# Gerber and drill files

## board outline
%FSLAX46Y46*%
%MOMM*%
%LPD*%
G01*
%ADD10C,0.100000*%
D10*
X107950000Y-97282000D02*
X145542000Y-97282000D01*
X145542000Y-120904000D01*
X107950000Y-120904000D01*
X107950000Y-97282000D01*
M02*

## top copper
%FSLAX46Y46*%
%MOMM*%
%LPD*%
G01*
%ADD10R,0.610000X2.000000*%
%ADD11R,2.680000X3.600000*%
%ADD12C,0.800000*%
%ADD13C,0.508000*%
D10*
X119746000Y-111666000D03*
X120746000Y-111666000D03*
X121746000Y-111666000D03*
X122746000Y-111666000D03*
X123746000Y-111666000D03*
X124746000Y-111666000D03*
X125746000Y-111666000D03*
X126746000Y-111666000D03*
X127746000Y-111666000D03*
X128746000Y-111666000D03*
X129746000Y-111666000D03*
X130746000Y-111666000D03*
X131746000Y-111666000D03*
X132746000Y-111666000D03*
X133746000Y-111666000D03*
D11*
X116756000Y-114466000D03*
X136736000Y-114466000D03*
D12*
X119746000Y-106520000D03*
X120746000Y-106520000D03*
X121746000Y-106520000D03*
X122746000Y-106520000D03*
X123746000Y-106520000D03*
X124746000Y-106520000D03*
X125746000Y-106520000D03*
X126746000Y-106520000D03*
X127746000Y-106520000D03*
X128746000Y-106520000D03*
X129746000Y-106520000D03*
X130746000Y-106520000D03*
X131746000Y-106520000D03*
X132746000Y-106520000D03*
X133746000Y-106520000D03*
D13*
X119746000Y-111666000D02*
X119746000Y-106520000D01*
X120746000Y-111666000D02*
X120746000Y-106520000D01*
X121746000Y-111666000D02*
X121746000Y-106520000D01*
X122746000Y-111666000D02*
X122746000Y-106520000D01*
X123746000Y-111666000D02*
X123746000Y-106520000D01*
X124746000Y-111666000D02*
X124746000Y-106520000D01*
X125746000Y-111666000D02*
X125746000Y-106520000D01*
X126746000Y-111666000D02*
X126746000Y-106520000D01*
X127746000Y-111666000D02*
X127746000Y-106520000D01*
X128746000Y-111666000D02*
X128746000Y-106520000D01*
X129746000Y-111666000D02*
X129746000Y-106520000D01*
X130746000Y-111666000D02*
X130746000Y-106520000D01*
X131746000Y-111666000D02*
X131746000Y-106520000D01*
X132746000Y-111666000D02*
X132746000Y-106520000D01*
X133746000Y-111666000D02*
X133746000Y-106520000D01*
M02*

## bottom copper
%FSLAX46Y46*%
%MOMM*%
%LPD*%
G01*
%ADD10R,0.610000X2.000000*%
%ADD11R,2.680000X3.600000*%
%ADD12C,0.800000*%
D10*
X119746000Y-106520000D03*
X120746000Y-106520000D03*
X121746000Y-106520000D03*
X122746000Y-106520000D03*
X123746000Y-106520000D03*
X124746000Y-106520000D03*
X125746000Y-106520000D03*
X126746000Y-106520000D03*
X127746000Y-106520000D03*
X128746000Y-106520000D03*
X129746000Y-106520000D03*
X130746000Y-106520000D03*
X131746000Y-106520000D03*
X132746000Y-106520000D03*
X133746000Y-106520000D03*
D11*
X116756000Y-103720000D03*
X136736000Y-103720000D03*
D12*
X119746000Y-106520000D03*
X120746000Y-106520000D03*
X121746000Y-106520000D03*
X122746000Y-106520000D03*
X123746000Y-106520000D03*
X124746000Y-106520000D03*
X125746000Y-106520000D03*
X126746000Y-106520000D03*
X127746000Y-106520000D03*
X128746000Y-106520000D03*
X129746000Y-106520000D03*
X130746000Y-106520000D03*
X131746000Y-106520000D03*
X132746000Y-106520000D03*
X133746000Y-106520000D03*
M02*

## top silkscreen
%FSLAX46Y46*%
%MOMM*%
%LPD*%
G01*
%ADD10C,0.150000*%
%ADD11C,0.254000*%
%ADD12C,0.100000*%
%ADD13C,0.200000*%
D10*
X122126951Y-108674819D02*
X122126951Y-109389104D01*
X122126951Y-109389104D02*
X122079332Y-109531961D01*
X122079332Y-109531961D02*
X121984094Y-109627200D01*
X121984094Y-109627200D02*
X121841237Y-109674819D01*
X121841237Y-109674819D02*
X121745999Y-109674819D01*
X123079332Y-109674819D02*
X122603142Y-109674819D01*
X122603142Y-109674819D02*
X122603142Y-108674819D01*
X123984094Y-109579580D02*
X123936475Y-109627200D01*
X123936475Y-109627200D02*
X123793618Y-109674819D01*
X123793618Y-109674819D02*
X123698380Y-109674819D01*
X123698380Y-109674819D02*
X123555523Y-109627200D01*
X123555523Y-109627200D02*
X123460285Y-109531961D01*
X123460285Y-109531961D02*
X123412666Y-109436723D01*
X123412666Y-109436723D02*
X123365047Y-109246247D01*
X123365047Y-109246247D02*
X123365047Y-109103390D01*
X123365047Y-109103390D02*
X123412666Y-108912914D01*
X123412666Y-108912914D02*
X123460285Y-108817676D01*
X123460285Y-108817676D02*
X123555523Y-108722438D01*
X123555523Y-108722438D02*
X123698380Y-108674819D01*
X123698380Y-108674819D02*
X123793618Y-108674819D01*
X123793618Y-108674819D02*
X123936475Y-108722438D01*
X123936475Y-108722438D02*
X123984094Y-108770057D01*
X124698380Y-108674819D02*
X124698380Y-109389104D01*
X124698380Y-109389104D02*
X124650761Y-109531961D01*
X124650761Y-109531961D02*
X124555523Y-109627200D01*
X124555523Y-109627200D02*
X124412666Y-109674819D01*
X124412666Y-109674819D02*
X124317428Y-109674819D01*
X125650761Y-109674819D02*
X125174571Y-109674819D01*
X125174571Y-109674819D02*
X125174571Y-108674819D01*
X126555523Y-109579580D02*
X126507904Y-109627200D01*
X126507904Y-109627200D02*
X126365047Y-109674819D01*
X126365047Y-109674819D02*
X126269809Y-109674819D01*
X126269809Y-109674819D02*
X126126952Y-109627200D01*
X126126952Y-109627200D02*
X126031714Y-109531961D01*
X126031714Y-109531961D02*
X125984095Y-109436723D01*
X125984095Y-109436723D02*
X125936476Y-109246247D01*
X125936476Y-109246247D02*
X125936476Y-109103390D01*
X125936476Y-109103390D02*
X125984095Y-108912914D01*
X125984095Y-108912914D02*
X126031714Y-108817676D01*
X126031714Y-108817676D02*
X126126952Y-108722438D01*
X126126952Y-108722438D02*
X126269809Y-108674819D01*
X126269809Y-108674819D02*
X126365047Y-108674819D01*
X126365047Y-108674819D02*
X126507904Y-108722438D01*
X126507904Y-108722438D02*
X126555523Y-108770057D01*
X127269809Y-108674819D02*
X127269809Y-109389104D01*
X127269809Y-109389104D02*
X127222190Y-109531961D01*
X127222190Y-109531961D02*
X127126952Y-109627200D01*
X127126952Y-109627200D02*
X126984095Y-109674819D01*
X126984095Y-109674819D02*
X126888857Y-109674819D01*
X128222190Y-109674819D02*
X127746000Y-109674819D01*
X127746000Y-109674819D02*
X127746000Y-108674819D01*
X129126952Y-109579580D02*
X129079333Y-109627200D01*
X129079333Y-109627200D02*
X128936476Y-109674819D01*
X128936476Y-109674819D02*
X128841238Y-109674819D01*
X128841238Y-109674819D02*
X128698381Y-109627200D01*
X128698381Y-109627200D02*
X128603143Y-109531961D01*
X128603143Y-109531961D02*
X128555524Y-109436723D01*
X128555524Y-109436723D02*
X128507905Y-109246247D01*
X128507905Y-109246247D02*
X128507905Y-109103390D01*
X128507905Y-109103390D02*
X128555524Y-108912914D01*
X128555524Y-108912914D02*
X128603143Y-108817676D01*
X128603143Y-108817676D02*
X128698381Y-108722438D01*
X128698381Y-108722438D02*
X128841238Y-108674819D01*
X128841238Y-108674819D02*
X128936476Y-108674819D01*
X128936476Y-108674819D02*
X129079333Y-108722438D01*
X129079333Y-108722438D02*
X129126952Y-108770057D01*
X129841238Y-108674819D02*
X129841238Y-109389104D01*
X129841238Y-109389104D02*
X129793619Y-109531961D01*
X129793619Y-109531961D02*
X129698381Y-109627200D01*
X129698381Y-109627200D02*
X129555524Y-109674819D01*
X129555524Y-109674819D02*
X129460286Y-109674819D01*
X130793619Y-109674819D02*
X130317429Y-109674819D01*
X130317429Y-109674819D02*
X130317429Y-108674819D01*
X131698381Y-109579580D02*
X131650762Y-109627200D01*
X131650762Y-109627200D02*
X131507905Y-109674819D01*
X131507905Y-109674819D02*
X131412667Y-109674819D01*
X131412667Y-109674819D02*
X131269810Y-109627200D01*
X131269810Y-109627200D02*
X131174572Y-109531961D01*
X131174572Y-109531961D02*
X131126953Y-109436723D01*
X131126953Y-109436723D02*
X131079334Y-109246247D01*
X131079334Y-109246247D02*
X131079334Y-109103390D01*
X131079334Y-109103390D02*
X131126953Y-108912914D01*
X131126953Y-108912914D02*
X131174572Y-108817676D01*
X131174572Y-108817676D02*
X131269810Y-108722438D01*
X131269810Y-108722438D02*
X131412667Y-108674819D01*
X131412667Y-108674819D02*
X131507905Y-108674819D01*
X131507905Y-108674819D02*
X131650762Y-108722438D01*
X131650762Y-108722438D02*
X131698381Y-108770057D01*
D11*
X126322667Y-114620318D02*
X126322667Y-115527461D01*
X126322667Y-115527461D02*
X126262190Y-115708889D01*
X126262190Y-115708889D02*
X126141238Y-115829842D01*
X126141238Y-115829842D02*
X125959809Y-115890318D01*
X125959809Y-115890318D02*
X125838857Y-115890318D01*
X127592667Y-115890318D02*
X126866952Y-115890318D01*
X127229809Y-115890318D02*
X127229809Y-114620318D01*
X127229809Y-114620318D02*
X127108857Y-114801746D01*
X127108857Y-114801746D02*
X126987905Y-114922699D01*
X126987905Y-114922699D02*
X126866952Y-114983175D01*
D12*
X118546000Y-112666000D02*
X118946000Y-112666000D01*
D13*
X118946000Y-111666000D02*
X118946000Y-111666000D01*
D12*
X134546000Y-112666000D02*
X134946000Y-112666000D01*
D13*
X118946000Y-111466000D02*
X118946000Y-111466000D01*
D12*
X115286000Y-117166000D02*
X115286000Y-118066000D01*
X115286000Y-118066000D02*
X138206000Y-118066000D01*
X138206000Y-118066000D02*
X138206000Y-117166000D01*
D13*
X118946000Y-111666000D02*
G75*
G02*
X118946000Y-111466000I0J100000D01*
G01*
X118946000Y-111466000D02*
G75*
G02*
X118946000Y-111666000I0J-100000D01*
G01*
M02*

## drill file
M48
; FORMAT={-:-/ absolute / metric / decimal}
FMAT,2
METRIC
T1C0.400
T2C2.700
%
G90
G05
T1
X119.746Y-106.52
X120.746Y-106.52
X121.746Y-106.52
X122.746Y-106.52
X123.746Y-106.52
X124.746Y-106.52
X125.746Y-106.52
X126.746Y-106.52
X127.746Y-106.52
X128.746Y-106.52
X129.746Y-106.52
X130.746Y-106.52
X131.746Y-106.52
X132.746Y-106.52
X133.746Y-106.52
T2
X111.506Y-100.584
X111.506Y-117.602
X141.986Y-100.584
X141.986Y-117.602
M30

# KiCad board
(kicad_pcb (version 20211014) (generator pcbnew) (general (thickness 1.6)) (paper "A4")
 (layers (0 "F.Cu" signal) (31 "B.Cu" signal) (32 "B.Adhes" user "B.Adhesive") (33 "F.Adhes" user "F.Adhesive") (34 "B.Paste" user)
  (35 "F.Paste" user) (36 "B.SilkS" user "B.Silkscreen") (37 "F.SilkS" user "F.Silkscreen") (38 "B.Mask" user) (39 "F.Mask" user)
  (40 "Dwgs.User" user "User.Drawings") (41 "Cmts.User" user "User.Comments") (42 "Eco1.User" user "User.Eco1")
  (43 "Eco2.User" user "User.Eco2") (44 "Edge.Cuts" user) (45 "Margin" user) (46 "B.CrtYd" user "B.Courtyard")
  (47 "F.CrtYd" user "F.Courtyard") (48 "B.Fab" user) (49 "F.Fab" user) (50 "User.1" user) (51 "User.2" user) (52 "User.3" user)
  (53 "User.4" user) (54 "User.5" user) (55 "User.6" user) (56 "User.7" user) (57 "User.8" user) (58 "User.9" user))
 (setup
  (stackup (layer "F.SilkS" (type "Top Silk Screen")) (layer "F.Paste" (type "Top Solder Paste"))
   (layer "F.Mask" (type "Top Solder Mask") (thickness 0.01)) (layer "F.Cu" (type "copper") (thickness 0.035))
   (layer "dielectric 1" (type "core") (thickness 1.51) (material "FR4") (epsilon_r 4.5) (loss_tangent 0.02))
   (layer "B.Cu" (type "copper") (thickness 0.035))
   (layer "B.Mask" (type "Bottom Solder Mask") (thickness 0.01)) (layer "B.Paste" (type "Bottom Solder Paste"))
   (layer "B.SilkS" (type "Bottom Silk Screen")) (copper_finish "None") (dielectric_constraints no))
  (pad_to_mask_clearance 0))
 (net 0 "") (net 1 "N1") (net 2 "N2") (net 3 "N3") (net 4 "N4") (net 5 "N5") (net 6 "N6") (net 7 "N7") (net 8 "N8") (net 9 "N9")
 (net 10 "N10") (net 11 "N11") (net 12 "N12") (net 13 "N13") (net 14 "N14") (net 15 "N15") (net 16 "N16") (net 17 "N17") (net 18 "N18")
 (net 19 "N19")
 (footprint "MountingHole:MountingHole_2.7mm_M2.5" (layer "F.Cu") (at 141.986 100.584)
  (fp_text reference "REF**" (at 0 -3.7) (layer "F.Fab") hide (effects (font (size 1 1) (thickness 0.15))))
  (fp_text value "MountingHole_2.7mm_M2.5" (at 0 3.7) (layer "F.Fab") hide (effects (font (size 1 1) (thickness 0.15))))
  (pad "" np_thru_hole circle locked (at 0 0) (size 2.7 2.7) (drill 2.7) (layers *.Cu *.Mask)))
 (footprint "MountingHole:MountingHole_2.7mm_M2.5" (layer "F.Cu") (at 141.986 117.602)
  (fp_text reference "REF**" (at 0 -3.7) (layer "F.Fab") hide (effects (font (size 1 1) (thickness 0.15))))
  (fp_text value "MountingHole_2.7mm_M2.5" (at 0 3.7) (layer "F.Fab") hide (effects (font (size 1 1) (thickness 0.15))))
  (pad "" np_thru_hole circle locked (at 0 0) (size 2.7 2.7) (drill 2.7) (layers *.Cu *.Mask)))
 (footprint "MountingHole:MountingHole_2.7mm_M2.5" (layer "F.Cu") (at 111.506 100.584)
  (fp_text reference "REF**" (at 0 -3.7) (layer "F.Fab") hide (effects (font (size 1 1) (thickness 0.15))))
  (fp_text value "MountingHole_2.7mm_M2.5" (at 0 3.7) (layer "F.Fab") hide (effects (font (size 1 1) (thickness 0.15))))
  (pad "" np_thru_hole circle locked (at 0 0) (size 2.7 2.7) (drill 2.7) (layers *.Cu *.Mask)))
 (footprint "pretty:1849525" (layer "F.Cu") (at 126.746 115.316)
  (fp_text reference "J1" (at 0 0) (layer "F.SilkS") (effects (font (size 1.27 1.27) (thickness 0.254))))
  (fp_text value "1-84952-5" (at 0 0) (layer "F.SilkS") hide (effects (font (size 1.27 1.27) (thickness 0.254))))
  (fp_line (start -8.2 -2.65) (end -7.8 -2.65) (layer "F.SilkS") (width 0.1))
  (fp_line (start -7.8 -3.65) (end -7.8 -3.65) (layer "F.SilkS") (width 0.2))
  (fp_line (start 7.8 -2.65) (end 8.2 -2.65) (layer "F.SilkS") (width 0.1))
  (fp_line (start -7.8 -3.85) (end -7.8 -3.85) (layer "F.SilkS") (width 0.2))
  (fp_line (start -11.46 1.85) (end -11.46 2.75) (layer "F.SilkS") (width 0.1))
  (fp_line (start -11.46 2.75) (end 11.46 2.75) (layer "F.SilkS") (width 0.1))
  (fp_line (start 11.46 2.75) (end 11.46 1.85) (layer "F.SilkS") (width 0.1))
  (fp_arc (start -7.8 -3.65) (mid -7.9 -3.75) (end -7.8 -3.85) (layer "F.SilkS") (width 0.2))
  (fp_arc (start -7.8 -3.85) (mid -7.7 -3.75) (end -7.8 -3.65) (layer "F.SilkS") (width 0.2))
  (pad "1" smd rect locked (at -7 -3.65) (size 0.61 2) (layers "F.Cu" "F.Paste" "F.Mask") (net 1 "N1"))
  (pad "2" smd rect locked (at -6 -3.65) (size 0.61 2) (layers "F.Cu" "F.Paste" "F.Mask") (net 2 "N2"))
  (pad "3" smd rect locked (at -5 -3.65) (size 0.61 2) (layers "F.Cu" "F.Paste" "F.Mask") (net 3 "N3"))
  (pad "4" smd rect locked (at -4 -3.65) (size 0.61 2) (layers "F.Cu" "F.Paste" "F.Mask") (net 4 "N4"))
  (pad "5" smd rect locked (at -3 -3.65) (size 0.61 2) (layers "F.Cu" "F.Paste" "F.Mask") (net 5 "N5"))
  (pad "6" smd rect locked (at -2 -3.65) (size 0.61 2) (layers "F.Cu" "F.Paste" "F.Mask") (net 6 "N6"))
  (pad "7" smd rect locked (at -1 -3.65) (size 0.61 2) (layers "F.Cu" "F.Paste" "F.Mask") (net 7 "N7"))
  (pad "8" smd rect locked (at 0 -3.65) (size 0.61 2) (layers "F.Cu" "F.Paste" "F.Mask") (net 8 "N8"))
  (pad "9" smd rect locked (at 1 -3.65) (size 0.61 2) (layers "F.Cu" "F.Paste" "F.Mask") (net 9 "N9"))
  (pad "10" smd rect locked (at 2 -3.65) (size 0.61 2) (layers "F.Cu" "F.Paste" "F.Mask") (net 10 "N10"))
  (pad "11" smd rect locked (at 3 -3.65) (size 0.61 2) (layers "F.Cu" "F.Paste" "F.Mask") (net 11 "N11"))
  (pad "12" smd rect locked (at 4 -3.65) (size 0.61 2) (layers "F.Cu" "F.Paste" "F.Mask") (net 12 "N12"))
  (pad "13" smd rect locked (at 5 -3.65) (size 0.61 2) (layers "F.Cu" "F.Paste" "F.Mask") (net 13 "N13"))
  (pad "14" smd rect locked (at 6 -3.65) (size 0.61 2) (layers "F.Cu" "F.Paste" "F.Mask") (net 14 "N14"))
  (pad "15" smd rect locked (at 7 -3.65) (size 0.61 2) (layers "F.Cu" "F.Paste" "F.Mask") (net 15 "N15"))
  (pad "MP1" smd rect locked (at -9.99 -0.85) (size 2.68 3.6) (layers "F.Cu" "F.Paste" "F.Mask") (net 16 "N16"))
  (pad "MP2" smd rect locked (at 9.99 -0.85) (size 2.68 3.6) (layers "F.Cu" "F.Paste" "F.Mask") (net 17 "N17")))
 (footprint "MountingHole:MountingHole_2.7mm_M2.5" (layer "F.Cu") (at 111.506 117.602)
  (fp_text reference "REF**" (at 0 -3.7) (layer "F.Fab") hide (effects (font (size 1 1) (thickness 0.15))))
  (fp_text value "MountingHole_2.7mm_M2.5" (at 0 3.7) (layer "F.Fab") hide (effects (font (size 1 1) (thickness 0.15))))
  (pad "" np_thru_hole circle locked (at 0 0) (size 2.7 2.7) (drill 2.7) (layers *.Cu *.Mask)))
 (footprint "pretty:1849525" (layer "B.Cu") (at 126.746 102.87)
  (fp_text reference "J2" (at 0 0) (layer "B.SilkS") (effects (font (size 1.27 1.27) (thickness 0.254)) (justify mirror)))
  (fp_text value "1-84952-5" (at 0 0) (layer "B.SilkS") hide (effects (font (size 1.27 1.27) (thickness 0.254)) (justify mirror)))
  (pad "1" smd rect locked (at -7 3.65) (size 0.61 2) (layers "B.Cu" "B.Paste" "B.Mask") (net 1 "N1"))
  (pad "2" smd rect locked (at -6 3.65) (size 0.61 2) (layers "B.Cu" "B.Paste" "B.Mask") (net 2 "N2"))
  (pad "3" smd rect locked (at -5 3.65) (size 0.61 2) (layers "B.Cu" "B.Paste" "B.Mask") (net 3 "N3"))
  (pad "4" smd rect locked (at -4 3.65) (size 0.61 2) (layers "B.Cu" "B.Paste" "B.Mask") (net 4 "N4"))
  (pad "5" smd rect locked (at -3 3.65) (size 0.61 2) (layers "B.Cu" "B.Paste" "B.Mask") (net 5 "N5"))
  (pad "6" smd rect locked (at -2 3.65) (size 0.61 2) (layers "B.Cu" "B.Paste" "B.Mask") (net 6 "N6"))
  (pad "7" smd rect locked (at -1 3.65) (size 0.61 2) (layers "B.Cu" "B.Paste" "B.Mask") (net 7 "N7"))
  (pad "8" smd rect locked (at 0 3.65) (size 0.61 2) (layers "B.Cu" "B.Paste" "B.Mask") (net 8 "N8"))
  (pad "9" smd rect locked (at 1 3.65) (size 0.61 2) (layers "B.Cu" "B.Paste" "B.Mask") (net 9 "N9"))
  (pad "10" smd rect locked (at 2 3.65) (size 0.61 2) (layers "B.Cu" "B.Paste" "B.Mask") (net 10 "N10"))
  (pad "11" smd rect locked (at 3 3.65) (size 0.61 2) (layers "B.Cu" "B.Paste" "B.Mask") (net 11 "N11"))
  (pad "12" smd rect locked (at 4 3.65) (size 0.61 2) (layers "B.Cu" "B.Paste" "B.Mask") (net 12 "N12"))
  (pad "13" smd rect locked (at 5 3.65) (size 0.61 2) (layers "B.Cu" "B.Paste" "B.Mask") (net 13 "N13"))
  (pad "14" smd rect locked (at 6 3.65) (size 0.61 2) (layers "B.Cu" "B.Paste" "B.Mask") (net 14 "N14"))
  (pad "15" smd rect locked (at 7 3.65) (size 0.61 2) (layers "B.Cu" "B.Paste" "B.Mask") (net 15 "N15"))
  (pad "MP1" smd rect locked (at -9.99 0.85) (size 2.68 3.6) (layers "B.Cu" "B.Paste" "B.Mask") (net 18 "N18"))
  (pad "MP2" smd rect locked (at 9.99 0.85) (size 2.68 3.6) (layers "B.Cu" "B.Paste" "B.Mask") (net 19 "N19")))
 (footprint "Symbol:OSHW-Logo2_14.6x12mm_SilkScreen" (layer "B.Cu") (at 126.746 114.046 180)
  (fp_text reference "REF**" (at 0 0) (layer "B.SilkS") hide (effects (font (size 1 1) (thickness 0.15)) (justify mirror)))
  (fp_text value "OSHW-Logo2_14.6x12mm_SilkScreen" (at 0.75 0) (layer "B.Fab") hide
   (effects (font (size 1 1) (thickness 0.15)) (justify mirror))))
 (gr_rect (start 145.542 97.282) (end 107.95 120.904) (layer "Edge.Cuts") (width 0.1) (fill none))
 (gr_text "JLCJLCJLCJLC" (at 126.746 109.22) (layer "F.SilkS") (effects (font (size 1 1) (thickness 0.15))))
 (segment (start 119.746 111.666) (end 119.746 106.52) (width 0.508) (layer "F.Cu") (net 1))
 (via (at 119.746 106.52) (size 0.8) (drill 0.4) (layers "F.Cu" "B.Cu") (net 1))
 (segment (start 120.746 111.666) (end 120.746 106.52) (width 0.508) (layer "F.Cu") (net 2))
 (via (at 120.746 106.52) (size 0.8) (drill 0.4) (layers "F.Cu" "B.Cu") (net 2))
 (segment (start 121.746 111.666) (end 121.746 106.52) (width 0.508) (layer "F.Cu") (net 3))
 (via (at 121.746 106.52) (size 0.8) (drill 0.4) (layers "F.Cu" "B.Cu") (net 3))
 (segment (start 122.746 111.666) (end 122.746 106.52) (width 0.508) (layer "F.Cu") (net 4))
 (via (at 122.746 106.52) (size 0.8) (drill 0.4) (layers "F.Cu" "B.Cu") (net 4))
 (segment (start 123.746 111.666) (end 123.746 106.52) (width 0.508) (layer "F.Cu") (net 5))
 (via (at 123.746 106.52) (size 0.8) (drill 0.4) (layers "F.Cu" "B.Cu") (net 5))
 (segment (start 124.746 111.666) (end 124.746 106.52) (width 0.508) (layer "F.Cu") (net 6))
 (via (at 124.746 106.52) (size 0.8) (drill 0.4) (layers "F.Cu" "B.Cu") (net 6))
 (segment (start 125.746 111.666) (end 125.746 106.52) (width 0.508) (layer "F.Cu") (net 7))
 (via (at 125.746 106.52) (size 0.8) (drill 0.4) (layers "F.Cu" "B.Cu") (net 7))
 (segment (start 126.746 111.666) (end 126.746 106.52) (width 0.508) (layer "F.Cu") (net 8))
 (via (at 126.746 106.52) (size 0.8) (drill 0.4) (layers "F.Cu" "B.Cu") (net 8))
 (segment (start 127.746 111.666) (end 127.746 106.52) (width 0.508) (layer "F.Cu") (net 9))
 (via (at 127.746 106.52) (size 0.8) (drill 0.4) (layers "F.Cu" "B.Cu") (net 9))
 (segment (start 128.746 111.666) (end 128.746 106.52) (width 0.508) (layer "F.Cu") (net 10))
 (via (at 128.746 106.52) (size 0.8) (drill 0.4) (layers "F.Cu" "B.Cu") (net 10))
 (segment (start 129.746 111.666) (end 129.746 106.52) (width 0.508) (layer "F.Cu") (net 11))
 (via (at 129.746 106.52) (size 0.8) (drill 0.4) (layers "F.Cu" "B.Cu") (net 11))
 (segment (start 130.746 111.666) (end 130.746 106.52) (width 0.508) (layer "F.Cu") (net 12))
 (via (at 130.746 106.52) (size 0.8) (drill 0.4) (layers "F.Cu" "B.Cu") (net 12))
 (segment (start 131.746 111.666) (end 131.746 106.52) (width 0.508) (layer "F.Cu") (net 13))
 (via (at 131.746 106.52) (size 0.8) (drill 0.4) (layers "F.Cu" "B.Cu") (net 13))
 (segment (start 132.746 111.666) (end 132.746 106.52) (width 0.508) (layer "F.Cu") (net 14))
 (via (at 132.746 106.52) (size 0.8) (drill 0.4) (layers "F.Cu" "B.Cu") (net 14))
 (segment (start 133.746 111.666) (end 133.746 106.52) (width 0.508) (layer "F.Cu") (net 15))
 (via (at 133.746 106.52) (size 0.8) (drill 0.4) (layers "F.Cu" "B.Cu") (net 15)))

